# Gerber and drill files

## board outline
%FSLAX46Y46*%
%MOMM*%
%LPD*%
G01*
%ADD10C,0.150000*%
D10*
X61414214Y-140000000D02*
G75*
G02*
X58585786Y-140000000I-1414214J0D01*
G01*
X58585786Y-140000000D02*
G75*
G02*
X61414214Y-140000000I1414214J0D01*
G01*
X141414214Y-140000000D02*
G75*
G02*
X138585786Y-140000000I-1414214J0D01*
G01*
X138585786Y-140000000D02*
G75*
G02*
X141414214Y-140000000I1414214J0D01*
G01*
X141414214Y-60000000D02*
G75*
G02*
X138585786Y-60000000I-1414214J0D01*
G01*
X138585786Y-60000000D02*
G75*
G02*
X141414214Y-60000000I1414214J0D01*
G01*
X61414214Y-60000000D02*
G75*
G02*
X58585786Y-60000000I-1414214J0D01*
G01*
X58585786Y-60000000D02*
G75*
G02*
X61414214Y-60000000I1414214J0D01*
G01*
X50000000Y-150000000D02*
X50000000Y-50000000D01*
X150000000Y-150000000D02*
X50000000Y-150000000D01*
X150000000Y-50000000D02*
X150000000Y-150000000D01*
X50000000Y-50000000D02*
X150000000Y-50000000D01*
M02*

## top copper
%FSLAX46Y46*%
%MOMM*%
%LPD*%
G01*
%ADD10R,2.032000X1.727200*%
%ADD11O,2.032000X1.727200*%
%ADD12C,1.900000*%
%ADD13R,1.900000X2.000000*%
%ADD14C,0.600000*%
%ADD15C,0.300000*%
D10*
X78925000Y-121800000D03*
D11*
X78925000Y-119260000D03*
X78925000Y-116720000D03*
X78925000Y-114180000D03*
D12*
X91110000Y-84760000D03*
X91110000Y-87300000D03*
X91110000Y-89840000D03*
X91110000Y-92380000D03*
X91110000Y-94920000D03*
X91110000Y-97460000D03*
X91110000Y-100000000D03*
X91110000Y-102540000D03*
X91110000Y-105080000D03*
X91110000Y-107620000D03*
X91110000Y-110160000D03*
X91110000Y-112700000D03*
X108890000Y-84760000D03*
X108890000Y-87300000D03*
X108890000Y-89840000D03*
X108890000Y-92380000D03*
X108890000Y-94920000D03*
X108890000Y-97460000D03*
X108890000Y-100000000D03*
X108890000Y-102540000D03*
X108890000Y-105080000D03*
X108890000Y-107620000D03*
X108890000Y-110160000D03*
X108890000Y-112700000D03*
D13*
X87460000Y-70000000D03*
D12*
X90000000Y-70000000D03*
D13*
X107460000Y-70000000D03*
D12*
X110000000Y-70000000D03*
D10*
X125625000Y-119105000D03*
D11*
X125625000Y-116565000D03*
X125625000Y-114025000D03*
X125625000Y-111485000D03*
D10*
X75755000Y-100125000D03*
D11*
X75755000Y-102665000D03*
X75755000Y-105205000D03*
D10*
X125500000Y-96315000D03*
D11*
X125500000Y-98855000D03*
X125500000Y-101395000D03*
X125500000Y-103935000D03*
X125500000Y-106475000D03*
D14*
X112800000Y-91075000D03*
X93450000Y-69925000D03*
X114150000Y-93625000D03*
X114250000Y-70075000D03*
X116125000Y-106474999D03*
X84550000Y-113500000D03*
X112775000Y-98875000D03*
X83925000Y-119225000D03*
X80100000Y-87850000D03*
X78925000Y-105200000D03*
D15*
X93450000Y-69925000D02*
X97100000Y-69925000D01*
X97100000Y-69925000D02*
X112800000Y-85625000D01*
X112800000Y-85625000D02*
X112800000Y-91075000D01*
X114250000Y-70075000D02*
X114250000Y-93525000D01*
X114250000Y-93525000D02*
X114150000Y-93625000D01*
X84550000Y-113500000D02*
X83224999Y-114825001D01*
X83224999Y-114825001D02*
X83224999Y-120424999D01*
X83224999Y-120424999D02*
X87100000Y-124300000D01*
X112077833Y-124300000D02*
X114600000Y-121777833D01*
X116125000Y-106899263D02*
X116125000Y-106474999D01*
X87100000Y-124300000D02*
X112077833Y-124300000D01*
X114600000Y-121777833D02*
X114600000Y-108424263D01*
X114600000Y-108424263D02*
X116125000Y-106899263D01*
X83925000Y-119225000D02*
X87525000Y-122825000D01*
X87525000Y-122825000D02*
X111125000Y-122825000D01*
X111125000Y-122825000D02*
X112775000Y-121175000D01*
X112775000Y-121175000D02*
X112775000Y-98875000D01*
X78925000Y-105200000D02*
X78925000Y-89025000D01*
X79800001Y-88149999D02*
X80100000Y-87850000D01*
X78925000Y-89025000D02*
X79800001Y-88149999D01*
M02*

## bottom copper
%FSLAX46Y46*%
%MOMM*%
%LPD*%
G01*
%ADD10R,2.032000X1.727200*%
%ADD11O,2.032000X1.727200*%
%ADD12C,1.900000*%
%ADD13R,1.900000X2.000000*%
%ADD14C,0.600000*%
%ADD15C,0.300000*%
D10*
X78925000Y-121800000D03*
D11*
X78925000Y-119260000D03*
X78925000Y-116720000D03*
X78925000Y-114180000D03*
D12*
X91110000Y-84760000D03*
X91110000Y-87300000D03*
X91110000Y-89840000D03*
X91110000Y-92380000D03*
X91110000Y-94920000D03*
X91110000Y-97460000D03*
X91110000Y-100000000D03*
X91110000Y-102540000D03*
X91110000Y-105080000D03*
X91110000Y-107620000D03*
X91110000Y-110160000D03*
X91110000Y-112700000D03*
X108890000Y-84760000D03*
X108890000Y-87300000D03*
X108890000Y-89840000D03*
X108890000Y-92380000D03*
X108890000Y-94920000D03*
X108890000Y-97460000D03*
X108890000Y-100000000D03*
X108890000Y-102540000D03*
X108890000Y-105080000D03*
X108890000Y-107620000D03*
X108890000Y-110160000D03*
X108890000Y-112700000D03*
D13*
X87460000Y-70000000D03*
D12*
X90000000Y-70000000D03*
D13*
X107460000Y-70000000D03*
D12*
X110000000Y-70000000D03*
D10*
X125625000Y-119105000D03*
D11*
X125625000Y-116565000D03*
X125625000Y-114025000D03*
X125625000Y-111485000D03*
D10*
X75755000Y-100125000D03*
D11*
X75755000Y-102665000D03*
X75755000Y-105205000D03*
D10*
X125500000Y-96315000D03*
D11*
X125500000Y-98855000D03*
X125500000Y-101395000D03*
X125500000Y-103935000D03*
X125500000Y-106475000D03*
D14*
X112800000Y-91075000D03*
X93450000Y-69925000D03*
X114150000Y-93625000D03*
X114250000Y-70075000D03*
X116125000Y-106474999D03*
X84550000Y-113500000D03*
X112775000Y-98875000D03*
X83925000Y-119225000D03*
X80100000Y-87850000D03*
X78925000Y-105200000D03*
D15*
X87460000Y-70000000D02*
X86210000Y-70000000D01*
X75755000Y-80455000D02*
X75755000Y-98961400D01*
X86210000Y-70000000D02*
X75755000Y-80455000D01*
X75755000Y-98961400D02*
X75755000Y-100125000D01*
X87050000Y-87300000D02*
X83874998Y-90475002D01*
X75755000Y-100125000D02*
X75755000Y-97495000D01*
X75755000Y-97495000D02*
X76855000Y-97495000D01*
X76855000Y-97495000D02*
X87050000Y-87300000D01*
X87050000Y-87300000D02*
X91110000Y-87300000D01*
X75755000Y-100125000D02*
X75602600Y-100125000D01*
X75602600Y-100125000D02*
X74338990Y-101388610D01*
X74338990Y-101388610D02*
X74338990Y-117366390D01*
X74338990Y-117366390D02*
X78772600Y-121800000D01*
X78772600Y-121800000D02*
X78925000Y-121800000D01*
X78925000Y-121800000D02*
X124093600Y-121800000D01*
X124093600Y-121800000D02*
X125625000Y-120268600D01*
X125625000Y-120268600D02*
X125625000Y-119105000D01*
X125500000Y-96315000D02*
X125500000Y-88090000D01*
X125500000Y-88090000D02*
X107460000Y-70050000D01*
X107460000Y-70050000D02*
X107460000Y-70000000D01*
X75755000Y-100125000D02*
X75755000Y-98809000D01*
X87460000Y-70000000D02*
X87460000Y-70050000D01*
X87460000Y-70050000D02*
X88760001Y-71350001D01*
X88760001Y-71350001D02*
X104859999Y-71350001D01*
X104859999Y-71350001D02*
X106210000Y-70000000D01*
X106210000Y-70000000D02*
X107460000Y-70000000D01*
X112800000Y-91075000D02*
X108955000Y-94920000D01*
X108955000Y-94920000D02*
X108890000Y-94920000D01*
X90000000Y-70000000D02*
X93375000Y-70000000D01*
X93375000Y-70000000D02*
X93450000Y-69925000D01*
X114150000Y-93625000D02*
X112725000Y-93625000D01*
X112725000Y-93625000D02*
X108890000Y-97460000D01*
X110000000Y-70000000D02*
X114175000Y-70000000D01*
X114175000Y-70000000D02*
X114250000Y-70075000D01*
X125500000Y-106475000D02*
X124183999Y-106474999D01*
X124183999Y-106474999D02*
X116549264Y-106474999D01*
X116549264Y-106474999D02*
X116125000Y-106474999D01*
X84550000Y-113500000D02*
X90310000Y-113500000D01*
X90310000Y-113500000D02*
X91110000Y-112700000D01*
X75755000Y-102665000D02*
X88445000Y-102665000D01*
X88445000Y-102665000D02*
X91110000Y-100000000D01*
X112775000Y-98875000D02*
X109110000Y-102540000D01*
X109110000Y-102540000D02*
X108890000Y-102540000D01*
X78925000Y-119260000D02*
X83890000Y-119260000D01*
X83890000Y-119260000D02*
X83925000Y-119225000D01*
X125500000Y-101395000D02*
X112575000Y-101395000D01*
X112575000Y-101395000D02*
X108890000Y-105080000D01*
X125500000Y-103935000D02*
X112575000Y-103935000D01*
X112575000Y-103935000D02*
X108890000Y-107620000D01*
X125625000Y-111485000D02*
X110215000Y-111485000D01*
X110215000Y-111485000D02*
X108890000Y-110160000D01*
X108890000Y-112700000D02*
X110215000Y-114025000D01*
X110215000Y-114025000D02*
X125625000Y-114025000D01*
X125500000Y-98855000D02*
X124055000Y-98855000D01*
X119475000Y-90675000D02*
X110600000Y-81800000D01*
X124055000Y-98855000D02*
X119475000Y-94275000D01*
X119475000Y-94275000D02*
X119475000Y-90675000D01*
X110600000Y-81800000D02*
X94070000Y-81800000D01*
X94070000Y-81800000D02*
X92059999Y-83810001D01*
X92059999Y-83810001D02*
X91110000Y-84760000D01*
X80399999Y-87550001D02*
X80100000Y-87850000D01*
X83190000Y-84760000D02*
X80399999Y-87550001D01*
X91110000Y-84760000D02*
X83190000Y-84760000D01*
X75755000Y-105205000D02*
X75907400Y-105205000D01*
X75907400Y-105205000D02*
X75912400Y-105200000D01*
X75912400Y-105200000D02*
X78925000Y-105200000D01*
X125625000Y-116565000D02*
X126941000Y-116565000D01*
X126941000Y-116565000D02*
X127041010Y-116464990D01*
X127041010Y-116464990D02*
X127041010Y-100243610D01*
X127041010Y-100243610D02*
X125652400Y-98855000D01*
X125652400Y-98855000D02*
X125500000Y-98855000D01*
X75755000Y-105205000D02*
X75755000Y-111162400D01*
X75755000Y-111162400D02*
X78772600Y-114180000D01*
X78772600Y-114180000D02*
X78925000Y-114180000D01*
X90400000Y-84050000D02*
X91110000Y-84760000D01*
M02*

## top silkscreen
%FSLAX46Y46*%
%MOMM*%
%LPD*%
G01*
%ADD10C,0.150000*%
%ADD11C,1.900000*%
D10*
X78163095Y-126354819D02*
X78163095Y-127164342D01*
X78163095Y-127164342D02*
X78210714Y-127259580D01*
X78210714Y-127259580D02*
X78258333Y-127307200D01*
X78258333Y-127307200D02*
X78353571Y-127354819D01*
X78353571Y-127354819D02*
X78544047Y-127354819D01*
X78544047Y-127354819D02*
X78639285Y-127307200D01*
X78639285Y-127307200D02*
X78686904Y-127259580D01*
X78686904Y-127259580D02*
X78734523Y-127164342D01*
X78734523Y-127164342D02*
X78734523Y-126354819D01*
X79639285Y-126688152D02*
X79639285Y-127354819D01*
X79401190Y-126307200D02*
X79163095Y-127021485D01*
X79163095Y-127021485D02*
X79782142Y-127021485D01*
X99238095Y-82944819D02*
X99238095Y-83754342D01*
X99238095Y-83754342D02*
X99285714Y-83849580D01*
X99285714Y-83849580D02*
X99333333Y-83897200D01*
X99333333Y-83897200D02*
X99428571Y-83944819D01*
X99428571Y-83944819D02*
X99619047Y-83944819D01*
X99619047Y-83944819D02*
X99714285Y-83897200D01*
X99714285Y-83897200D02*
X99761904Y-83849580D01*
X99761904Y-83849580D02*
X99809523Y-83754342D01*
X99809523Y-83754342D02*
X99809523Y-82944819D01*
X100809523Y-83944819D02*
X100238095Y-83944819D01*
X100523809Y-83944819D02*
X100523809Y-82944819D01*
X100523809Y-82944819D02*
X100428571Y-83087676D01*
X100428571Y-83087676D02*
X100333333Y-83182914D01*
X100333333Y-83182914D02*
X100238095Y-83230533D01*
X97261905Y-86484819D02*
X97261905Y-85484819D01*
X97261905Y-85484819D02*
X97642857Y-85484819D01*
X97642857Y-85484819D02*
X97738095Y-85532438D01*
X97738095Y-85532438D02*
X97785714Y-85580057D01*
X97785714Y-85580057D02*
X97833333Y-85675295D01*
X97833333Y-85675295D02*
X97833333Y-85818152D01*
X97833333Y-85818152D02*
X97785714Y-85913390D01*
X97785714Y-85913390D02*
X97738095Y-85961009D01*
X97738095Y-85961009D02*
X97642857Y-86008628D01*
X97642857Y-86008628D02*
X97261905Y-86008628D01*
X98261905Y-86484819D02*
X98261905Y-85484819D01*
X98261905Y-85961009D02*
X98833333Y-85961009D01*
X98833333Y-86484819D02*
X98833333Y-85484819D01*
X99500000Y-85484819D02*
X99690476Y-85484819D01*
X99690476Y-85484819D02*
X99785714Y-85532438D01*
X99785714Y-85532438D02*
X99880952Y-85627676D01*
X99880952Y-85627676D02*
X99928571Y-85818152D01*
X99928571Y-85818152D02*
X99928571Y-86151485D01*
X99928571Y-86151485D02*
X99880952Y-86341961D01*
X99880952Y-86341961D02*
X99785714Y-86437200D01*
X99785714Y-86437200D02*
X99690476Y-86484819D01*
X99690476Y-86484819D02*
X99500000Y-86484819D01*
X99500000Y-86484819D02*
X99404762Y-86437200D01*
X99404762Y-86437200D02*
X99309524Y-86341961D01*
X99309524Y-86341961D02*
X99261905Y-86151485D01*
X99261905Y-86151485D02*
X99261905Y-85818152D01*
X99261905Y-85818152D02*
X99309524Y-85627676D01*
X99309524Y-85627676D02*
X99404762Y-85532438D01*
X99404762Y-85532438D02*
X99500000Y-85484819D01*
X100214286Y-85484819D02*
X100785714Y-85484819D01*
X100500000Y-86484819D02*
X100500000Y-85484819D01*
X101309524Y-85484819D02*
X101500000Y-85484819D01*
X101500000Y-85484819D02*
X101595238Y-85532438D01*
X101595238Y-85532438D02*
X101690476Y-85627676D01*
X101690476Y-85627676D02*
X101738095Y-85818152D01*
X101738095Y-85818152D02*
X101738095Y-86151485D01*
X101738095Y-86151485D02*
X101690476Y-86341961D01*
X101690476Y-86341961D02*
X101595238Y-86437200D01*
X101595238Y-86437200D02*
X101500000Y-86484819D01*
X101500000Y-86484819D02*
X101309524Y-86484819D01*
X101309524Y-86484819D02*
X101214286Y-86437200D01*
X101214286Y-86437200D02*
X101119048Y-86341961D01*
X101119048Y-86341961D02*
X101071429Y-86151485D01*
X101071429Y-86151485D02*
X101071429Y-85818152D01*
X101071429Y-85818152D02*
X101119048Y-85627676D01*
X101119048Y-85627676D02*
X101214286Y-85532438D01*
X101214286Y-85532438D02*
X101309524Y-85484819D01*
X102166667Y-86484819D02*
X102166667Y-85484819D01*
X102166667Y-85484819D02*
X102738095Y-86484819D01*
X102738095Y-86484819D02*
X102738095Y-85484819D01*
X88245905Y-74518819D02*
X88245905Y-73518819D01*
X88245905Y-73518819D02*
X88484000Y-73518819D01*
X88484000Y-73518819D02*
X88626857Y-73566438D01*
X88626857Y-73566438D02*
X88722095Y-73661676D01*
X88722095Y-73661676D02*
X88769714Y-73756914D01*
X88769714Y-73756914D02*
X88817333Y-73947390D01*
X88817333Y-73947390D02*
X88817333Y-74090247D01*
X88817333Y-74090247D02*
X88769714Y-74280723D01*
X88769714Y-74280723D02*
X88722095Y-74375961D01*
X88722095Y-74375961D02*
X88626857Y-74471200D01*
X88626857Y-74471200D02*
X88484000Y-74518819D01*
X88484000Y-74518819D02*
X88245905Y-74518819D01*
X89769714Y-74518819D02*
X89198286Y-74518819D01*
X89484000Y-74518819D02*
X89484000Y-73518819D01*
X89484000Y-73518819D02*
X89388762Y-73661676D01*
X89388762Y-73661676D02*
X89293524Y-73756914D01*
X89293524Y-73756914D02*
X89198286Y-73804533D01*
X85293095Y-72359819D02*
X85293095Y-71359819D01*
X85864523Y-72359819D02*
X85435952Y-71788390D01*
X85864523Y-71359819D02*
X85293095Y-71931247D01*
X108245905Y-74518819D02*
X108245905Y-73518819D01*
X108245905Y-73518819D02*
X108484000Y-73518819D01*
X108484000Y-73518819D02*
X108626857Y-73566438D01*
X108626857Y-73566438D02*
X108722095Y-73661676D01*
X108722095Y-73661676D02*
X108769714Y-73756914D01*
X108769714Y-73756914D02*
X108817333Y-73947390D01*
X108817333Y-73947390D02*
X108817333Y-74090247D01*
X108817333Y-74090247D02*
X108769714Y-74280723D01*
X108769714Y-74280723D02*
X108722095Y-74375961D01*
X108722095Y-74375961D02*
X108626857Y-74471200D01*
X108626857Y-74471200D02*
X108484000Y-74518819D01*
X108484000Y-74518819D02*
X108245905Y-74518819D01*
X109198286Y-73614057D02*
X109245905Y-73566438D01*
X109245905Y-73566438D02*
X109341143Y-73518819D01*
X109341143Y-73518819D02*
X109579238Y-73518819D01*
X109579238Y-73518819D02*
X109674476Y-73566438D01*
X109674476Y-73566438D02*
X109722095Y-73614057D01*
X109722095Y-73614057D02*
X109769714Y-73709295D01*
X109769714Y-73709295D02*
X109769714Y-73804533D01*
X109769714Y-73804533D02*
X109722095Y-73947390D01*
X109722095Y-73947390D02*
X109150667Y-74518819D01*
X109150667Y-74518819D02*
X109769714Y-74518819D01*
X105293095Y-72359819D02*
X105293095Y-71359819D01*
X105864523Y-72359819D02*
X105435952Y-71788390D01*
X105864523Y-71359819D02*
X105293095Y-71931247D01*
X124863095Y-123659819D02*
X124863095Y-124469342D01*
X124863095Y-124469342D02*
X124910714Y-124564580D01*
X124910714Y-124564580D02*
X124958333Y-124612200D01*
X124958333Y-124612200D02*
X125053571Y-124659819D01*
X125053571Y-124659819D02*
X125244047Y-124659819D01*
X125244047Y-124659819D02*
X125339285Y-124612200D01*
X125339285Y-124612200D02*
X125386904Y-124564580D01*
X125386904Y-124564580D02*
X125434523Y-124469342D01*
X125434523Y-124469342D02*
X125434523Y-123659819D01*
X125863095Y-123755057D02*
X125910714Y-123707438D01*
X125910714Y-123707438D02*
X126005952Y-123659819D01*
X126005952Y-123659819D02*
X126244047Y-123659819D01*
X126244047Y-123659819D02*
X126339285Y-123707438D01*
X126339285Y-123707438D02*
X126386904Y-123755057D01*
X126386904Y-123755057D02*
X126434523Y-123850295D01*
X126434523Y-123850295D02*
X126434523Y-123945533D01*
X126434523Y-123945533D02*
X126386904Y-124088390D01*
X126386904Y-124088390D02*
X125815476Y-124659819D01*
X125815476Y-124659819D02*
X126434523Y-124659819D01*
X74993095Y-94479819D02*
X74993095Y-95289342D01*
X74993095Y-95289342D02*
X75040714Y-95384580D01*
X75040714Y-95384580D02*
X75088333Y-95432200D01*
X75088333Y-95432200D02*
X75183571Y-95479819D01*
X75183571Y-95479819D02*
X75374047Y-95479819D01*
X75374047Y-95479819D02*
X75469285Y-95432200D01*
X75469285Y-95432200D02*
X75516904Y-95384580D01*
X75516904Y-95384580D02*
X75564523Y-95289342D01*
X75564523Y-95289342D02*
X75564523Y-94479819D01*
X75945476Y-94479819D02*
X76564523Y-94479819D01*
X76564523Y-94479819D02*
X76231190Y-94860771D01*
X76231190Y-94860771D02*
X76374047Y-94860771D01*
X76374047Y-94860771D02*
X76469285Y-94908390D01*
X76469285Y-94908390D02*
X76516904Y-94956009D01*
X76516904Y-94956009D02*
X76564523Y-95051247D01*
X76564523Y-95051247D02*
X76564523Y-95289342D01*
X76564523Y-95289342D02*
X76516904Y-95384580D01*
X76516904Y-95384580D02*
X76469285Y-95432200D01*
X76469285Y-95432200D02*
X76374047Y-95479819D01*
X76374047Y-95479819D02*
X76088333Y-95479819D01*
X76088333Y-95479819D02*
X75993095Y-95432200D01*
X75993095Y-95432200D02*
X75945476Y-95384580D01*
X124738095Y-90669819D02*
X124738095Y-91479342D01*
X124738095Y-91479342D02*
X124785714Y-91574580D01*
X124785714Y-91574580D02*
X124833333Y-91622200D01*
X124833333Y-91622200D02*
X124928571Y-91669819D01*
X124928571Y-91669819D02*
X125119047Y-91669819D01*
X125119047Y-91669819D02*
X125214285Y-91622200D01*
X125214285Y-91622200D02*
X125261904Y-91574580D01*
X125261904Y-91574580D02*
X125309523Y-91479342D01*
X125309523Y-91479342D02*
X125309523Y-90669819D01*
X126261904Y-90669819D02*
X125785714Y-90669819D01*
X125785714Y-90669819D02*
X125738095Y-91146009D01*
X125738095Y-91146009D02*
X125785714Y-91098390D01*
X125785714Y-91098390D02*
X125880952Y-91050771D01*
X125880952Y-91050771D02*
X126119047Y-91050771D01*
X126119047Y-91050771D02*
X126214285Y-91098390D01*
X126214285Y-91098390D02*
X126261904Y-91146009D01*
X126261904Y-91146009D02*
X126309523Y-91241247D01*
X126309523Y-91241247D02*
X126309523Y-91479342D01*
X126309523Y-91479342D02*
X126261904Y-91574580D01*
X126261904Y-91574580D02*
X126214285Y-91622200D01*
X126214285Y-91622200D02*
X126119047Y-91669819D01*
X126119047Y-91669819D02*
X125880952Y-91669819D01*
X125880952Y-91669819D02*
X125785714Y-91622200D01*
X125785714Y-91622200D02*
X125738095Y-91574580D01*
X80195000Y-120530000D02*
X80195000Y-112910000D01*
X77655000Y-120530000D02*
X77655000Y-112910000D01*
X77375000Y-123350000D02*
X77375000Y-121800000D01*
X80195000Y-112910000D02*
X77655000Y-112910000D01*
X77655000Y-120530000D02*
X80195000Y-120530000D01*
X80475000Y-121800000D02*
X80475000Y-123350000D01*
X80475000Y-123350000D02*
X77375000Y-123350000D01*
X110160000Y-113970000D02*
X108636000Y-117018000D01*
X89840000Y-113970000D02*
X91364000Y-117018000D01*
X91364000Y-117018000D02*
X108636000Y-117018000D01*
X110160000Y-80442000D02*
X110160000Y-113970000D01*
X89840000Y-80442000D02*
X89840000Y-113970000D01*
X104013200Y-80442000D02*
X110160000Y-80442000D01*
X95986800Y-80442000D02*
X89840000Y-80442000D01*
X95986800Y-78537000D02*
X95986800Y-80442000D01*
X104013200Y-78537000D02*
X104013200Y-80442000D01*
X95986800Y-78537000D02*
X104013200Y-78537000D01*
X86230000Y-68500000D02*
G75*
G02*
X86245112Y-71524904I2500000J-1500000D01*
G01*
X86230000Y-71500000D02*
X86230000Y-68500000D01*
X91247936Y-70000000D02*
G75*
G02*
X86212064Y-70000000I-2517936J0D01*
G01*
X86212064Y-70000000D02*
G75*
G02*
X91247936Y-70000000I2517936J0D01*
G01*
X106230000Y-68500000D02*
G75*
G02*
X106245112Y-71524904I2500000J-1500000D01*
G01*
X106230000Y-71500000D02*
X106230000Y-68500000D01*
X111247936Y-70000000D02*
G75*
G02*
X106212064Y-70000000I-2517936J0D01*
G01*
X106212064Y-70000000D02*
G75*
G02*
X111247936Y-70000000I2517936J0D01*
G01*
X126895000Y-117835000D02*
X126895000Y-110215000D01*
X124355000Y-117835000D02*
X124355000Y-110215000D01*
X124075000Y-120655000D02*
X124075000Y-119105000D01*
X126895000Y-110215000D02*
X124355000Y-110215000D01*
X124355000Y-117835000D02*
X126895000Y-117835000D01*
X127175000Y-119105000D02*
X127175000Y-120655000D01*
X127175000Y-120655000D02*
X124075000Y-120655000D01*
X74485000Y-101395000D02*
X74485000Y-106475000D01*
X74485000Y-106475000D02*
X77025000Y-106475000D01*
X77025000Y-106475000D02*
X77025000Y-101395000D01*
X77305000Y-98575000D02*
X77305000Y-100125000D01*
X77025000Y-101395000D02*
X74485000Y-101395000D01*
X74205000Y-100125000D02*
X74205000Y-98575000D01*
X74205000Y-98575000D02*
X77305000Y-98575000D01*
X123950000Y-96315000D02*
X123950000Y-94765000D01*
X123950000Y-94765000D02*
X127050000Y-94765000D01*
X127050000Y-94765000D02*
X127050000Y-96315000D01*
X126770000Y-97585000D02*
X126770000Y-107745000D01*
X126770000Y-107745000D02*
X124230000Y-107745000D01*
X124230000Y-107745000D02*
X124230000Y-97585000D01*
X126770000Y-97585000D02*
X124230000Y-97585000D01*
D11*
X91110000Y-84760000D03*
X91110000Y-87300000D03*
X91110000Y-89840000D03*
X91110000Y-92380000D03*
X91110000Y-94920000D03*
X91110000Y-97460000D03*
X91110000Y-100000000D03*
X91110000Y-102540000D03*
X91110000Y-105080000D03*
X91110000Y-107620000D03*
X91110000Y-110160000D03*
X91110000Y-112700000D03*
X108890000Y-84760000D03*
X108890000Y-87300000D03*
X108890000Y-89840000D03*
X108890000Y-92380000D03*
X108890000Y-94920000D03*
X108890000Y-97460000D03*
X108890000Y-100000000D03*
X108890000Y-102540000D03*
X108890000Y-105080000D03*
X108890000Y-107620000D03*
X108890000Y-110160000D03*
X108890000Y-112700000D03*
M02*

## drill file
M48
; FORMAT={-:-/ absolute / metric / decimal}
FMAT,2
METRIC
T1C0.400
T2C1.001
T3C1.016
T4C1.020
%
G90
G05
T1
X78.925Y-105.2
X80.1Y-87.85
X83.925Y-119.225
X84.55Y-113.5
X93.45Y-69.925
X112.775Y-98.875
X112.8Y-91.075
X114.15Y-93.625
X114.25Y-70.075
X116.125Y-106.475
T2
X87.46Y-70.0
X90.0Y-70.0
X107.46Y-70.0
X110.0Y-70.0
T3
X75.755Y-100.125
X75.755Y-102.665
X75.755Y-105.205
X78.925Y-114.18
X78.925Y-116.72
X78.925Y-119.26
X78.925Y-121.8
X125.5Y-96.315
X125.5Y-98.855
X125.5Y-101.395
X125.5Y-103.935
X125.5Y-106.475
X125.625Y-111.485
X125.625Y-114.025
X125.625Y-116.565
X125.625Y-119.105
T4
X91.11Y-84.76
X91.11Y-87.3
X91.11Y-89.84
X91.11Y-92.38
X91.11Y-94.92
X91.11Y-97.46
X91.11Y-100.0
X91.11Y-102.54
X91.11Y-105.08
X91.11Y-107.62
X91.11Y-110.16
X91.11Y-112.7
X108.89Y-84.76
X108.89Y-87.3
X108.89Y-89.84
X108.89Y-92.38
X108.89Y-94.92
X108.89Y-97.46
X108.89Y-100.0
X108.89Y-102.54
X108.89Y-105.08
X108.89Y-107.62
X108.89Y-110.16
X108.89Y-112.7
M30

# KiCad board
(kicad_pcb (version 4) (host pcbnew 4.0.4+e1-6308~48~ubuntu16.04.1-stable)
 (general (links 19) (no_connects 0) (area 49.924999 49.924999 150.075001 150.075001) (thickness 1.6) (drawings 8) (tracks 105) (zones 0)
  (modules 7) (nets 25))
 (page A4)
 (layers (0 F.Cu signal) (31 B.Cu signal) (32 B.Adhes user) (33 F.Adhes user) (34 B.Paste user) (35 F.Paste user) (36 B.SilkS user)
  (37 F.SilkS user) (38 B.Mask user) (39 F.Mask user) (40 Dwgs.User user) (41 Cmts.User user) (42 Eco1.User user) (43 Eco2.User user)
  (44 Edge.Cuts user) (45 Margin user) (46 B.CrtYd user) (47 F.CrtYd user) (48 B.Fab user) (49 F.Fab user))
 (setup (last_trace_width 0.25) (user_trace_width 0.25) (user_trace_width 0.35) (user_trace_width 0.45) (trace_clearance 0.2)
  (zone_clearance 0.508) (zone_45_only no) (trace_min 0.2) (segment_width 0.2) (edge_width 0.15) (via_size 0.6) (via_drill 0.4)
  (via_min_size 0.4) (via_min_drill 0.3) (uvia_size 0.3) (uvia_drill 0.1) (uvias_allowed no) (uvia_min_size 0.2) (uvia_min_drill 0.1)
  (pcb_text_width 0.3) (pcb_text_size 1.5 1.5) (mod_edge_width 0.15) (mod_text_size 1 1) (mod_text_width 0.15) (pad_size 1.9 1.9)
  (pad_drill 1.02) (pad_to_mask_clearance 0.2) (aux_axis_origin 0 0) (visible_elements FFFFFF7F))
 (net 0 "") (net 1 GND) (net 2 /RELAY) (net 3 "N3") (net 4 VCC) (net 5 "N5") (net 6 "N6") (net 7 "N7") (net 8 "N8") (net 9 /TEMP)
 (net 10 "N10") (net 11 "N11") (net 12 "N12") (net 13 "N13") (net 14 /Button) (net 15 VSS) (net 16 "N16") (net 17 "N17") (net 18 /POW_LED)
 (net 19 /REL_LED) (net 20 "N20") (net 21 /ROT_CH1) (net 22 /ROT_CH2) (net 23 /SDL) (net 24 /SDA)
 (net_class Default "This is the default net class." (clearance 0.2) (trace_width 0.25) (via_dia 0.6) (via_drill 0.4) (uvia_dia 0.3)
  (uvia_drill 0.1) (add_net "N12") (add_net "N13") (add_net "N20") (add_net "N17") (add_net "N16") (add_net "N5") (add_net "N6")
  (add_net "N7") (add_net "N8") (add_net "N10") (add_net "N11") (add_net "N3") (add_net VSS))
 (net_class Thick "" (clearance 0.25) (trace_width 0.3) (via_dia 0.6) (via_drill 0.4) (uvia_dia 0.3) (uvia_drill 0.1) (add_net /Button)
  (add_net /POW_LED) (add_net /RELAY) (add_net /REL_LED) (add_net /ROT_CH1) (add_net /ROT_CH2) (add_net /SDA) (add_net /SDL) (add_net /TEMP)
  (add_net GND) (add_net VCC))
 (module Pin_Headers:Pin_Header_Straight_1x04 (layer F.Cu) (at 78.925 121.8 180)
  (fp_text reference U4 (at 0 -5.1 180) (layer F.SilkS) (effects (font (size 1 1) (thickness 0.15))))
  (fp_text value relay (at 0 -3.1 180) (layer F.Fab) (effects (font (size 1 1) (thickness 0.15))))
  (fp_line (start -1.27 1.27) (end -1.27 8.89) (layer F.SilkS) (width 0.15))
  (fp_line (start 1.27 1.27) (end 1.27 8.89) (layer F.SilkS) (width 0.15))
  (fp_line (start 1.55 -1.55) (end 1.55 0) (layer F.SilkS) (width 0.15))
  (fp_line (start -1.27 8.89) (end 1.27 8.89) (layer F.SilkS) (width 0.15))
  (fp_line (start 1.27 1.27) (end -1.27 1.27) (layer F.SilkS) (width 0.15))
  (fp_line (start -1.55 0) (end -1.55 -1.55) (layer F.SilkS) (width 0.15))
  (fp_line (start -1.55 -1.55) (end 1.55 -1.55) (layer F.SilkS) (width 0.15))
  (pad 1 thru_hole rect (at 0 0 180) (size 2.032 1.7272) (drill 1.016) (layers *.Cu *.Mask) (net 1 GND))
  (pad 2 thru_hole oval (at 0 2.54 180) (size 2.032 1.7272) (drill 1.016) (layers *.Cu *.Mask) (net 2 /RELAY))
  (pad 3 thru_hole oval (at 0 5.08 180) (size 2.032 1.7272) (drill 1.016) (layers *.Cu *.Mask) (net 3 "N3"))
  (pad 4 thru_hole oval (at 0 7.62 180) (size 2.032 1.7272) (drill 1.016) (layers *.Cu *.Mask) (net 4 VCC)))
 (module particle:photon (layer F.Cu) (at 100 100)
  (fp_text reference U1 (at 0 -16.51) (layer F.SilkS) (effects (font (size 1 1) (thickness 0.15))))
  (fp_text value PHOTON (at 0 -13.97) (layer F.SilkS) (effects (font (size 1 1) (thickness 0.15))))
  (fp_line (start 10.16 13.97) (end 8.636 17.018) (layer F.SilkS) (width 0.15))
  (fp_line (start -10.16 13.97) (end -8.636 17.018) (layer F.SilkS) (width 0.15))
  (fp_line (start -8.636 17.018) (end 8.636 17.018) (layer F.SilkS) (width 0.15))
  (fp_line (start 10.16 -19.558) (end 10.16 13.97) (layer F.SilkS) (width 0.15))
  (fp_line (start -10.16 -19.558) (end -10.16 13.97) (layer F.SilkS) (width 0.15))
  (fp_line (start 4.0132 -19.558) (end 10.16 -19.558) (layer F.SilkS) (width 0.15))
  (fp_line (start -4.0132 -19.558) (end -10.16 -19.558) (layer F.SilkS) (width 0.15))
  (fp_line (start -4.0132 -21.463) (end -4.0132 -19.558) (layer F.SilkS) (width 0.15))
  (fp_line (start 4.0132 -21.463) (end 4.0132 -19.558) (layer F.SilkS) (width 0.15))
  (fp_line (start -4.0132 -21.463) (end 4.0132 -21.463) (layer F.SilkS) (width 0.15))
  (pad 1 thru_hole circle (at -8.89 -15.24) (size 1.9 1.9) (drill 1.02) (layers *.Cu *.Mask F.SilkS) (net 4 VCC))
  (pad 2 thru_hole circle (at -8.89 -12.7) (size 1.9 1.9) (drill 1.02) (layers *.Cu *.Mask F.SilkS) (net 1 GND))
  (pad 3 thru_hole circle (at -8.89 -10.16) (size 1.9 1.9) (drill 1.02) (layers *.Cu *.Mask F.SilkS) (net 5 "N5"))
  (pad 4 thru_hole circle (at -8.89 -7.62) (size 1.9 1.9) (drill 1.02) (layers *.Cu *.Mask F.SilkS) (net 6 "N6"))
  (pad 5 thru_hole circle (at -8.89 -5.08) (size 1.9 1.9) (drill 1.02) (layers *.Cu *.Mask F.SilkS) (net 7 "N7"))
  (pad 6 thru_hole circle (at -8.89 -2.54) (size 1.9 1.9) (drill 1.02) (layers *.Cu *.Mask F.SilkS) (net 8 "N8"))
  (pad 7 thru_hole circle (at -8.89 0) (size 1.9 1.9) (drill 1.02) (layers *.Cu *.Mask F.SilkS) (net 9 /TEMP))
  (pad 8 thru_hole circle (at -8.89 2.54) (size 1.9 1.9) (drill 1.02) (layers *.Cu *.Mask F.SilkS) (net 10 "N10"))
  (pad 9 thru_hole circle (at -8.89 5.08) (size 1.9 1.9) (drill 1.02) (layers *.Cu *.Mask F.SilkS) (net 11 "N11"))
  (pad 10 thru_hole circle (at -8.89 7.62) (size 1.9 1.9) (drill 1.02) (layers *.Cu *.Mask F.SilkS) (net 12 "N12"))
  (pad 11 thru_hole circle (at -8.89 10.16) (size 1.9 1.9) (drill 1.02) (layers *.Cu *.Mask F.SilkS) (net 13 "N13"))
  (pad 12 thru_hole circle (at -8.89 12.7) (size 1.9 1.9) (drill 1.02) (layers *.Cu *.Mask F.SilkS) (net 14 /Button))
  (pad 24 thru_hole circle (at 8.89 -15.24) (size 1.9 1.9) (drill 1.02) (layers *.Cu *.Mask F.SilkS) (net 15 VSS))
  (pad 23 thru_hole circle (at 8.89 -12.7) (size 1.9 1.9) (drill 1.02) (layers *.Cu *.Mask F.SilkS) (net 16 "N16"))
  (pad 22 thru_hole circle (at 8.89 -10.16) (size 1.9 1.9) (drill 1.02) (layers *.Cu *.Mask F.SilkS) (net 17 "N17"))
  (pad 21 thru_hole circle (at 8.89 -7.62) (size 1.9 1.9) (drill 1.02) (layers *.Cu *.Mask F.SilkS))
  (pad 20 thru_hole circle (at 8.89 -5.08) (size 1.9 1.9) (drill 1.02) (layers *.Cu *.Mask F.SilkS) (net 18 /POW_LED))
  (pad 19 thru_hole circle (at 8.89 -2.54) (size 1.9 1.9) (drill 1.02) (layers *.Cu *.Mask F.SilkS) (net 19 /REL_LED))
  (pad 18 thru_hole circle (at 8.89 0) (size 1.9 1.9) (drill 1.02) (layers *.Cu *.Mask F.SilkS) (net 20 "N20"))
  (pad 17 thru_hole circle (at 8.89 2.54) (size 1.9 1.9) (drill 1.02) (layers *.Cu *.Mask F.SilkS) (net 2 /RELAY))
  (pad 16 thru_hole circle (at 8.89 5.08) (size 1.9 1.9) (drill 1.02) (layers *.Cu *.Mask F.SilkS) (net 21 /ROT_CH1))
  (pad 15 thru_hole circle (at 8.89 7.62) (size 1.9 1.9) (drill 1.02) (layers *.Cu *.Mask F.SilkS) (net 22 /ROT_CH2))
  (pad 14 thru_hole circle (at 8.89 10.16) (size 1.9 1.9) (drill 1.02) (layers *.Cu *.Mask F.SilkS) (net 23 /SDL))
  (pad 13 thru_hole circle (at 8.89 12.7) (size 1.9 1.9) (drill 1.02) (layers *.Cu *.Mask F.SilkS) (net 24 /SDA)))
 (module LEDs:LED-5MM (layer F.Cu) (at 87.46 70)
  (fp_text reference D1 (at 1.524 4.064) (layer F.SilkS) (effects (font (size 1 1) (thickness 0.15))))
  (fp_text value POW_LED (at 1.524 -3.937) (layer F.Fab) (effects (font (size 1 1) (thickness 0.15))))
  (fp_arc (start 1.27 0) (end -1.23 -1.5) (angle 297.5) (layer F.SilkS) (width 0.15))
  (fp_line (start -1.23 1.5) (end -1.23 -1.5) (layer F.SilkS) (width 0.15))
  (fp_circle (center 1.27 0) (end 0.97 -2.5) (layer F.SilkS) (width 0.15))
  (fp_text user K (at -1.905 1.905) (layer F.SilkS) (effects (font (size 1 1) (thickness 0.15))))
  (pad 1 thru_hole rect (at 0 0 90) (size 2 1.9) (drill 1.00076) (layers *.Cu *.Mask) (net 1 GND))
  (pad 2 thru_hole circle (at 2.54 0) (size 1.9 1.9) (drill 1.00076) (layers *.Cu *.Mask) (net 18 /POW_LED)))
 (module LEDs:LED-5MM (layer F.Cu) (at 107.46 70)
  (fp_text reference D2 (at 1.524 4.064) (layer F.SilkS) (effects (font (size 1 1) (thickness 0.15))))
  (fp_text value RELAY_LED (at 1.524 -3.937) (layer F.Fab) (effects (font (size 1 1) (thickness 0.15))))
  (fp_arc (start 1.27 0) (end -1.23 -1.5) (angle 297.5) (layer F.SilkS) (width 0.15))
  (fp_line (start -1.23 1.5) (end -1.23 -1.5) (layer F.SilkS) (width 0.15))
  (fp_circle (center 1.27 0) (end 0.97 -2.5) (layer F.SilkS) (width 0.15))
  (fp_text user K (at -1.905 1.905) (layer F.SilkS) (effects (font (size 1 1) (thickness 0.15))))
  (pad 1 thru_hole rect (at 0 0 90) (size 2 1.9) (drill 1.00076) (layers *.Cu *.Mask) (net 1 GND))
  (pad 2 thru_hole circle (at 2.54 0) (size 1.9 1.9) (drill 1.00076) (layers *.Cu *.Mask) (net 19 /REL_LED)))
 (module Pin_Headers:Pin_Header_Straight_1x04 (layer F.Cu) (at 125.625 119.105 180)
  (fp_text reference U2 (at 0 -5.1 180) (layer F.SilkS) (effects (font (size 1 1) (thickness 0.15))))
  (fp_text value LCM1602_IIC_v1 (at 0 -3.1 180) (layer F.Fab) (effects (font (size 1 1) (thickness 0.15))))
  (fp_line (start -1.27 1.27) (end -1.27 8.89) (layer F.SilkS) (width 0.15))
  (fp_line (start 1.27 1.27) (end 1.27 8.89) (layer F.SilkS) (width 0.15))
  (fp_line (start 1.55 -1.55) (end 1.55 0) (layer F.SilkS) (width 0.15))
  (fp_line (start -1.27 8.89) (end 1.27 8.89) (layer F.SilkS) (width 0.15))
  (fp_line (start 1.27 1.27) (end -1.27 1.27) (layer F.SilkS) (width 0.15))
  (fp_line (start -1.55 0) (end -1.55 -1.55) (layer F.SilkS) (width 0.15))
  (fp_line (start -1.55 -1.55) (end 1.55 -1.55) (layer F.SilkS) (width 0.15))
  (pad 1 thru_hole rect (at 0 0 180) (size 2.032 1.7272) (drill 1.016) (layers *.Cu *.Mask) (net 1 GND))
  (pad 2 thru_hole oval (at 0 2.54 180) (size 2.032 1.7272) (drill 1.016) (layers *.Cu *.Mask) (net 4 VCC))
  (pad 3 thru_hole oval (at 0 5.08 180) (size 2.032 1.7272) (drill 1.016) (layers *.Cu *.Mask) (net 24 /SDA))
  (pad 4 thru_hole oval (at 0 7.62 180) (size 2.032 1.7272) (drill 1.016) (layers *.Cu *.Mask) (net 23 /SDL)))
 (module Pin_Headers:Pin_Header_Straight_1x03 (layer F.Cu) (at 75.755 100.125)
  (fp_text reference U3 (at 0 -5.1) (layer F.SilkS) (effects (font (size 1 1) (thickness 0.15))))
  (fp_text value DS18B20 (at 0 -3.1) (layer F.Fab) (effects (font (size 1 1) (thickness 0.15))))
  (fp_line (start -1.27 1.27) (end -1.27 6.35) (layer F.SilkS) (width 0.15))
  (fp_line (start -1.27 6.35) (end 1.27 6.35) (layer F.SilkS) (width 0.15))
  (fp_line (start 1.27 6.35) (end 1.27 1.27) (layer F.SilkS) (width 0.15))
  (fp_line (start 1.55 -1.55) (end 1.55 0) (layer F.SilkS) (width 0.15))
  (fp_line (start 1.27 1.27) (end -1.27 1.27) (layer F.SilkS) (width 0.15))
  (fp_line (start -1.55 0) (end -1.55 -1.55) (layer F.SilkS) (width 0.15))
  (fp_line (start -1.55 -1.55) (end 1.55 -1.55) (layer F.SilkS) (width 0.15))
  (pad 1 thru_hole rect (at 0 0) (size 2.032 1.7272) (drill 1.016) (layers *.Cu *.Mask) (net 1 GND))
  (pad 2 thru_hole oval (at 0 2.54) (size 2.032 1.7272) (drill 1.016) (layers *.Cu *.Mask) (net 9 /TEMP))
  (pad 3 thru_hole oval (at 0 5.08) (size 2.032 1.7272) (drill 1.016) (layers *.Cu *.Mask) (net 4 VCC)))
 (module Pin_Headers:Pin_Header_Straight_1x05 (layer F.Cu) (at 125.5 96.315)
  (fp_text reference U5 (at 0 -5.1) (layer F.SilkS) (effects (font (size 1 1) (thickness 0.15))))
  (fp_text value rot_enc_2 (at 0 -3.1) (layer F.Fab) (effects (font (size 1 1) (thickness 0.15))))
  (fp_line (start -1.55 0) (end -1.55 -1.55) (layer F.SilkS) (width 0.15))
  (fp_line (start -1.55 -1.55) (end 1.55 -1.55) (layer F.SilkS) (width 0.15))
  (fp_line (start 1.55 -1.55) (end 1.55 0) (layer F.SilkS) (width 0.15))
  (fp_line (start 1.27 1.27) (end 1.27 11.43) (layer F.SilkS) (width 0.15))
  (fp_line (start 1.27 11.43) (end -1.27 11.43) (layer F.SilkS) (width 0.15))
  (fp_line (start -1.27 11.43) (end -1.27 1.27) (layer F.SilkS) (width 0.15))
  (fp_line (start 1.27 1.27) (end -1.27 1.27) (layer F.SilkS) (width 0.15))
  (pad 1 thru_hole rect (at 0 0) (size 2.032 1.7272) (drill 1.016) (layers *.Cu *.Mask) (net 1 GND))
  (pad 2 thru_hole oval (at 0 2.54) (size 2.032 1.7272) (drill 1.016) (layers *.Cu *.Mask) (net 4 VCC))
  (pad 3 thru_hole oval (at 0 5.08) (size 2.032 1.7272) (drill 1.016) (layers *.Cu *.Mask) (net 21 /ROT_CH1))
  (pad 4 thru_hole oval (at 0 7.62) (size 2.032 1.7272) (drill 1.016) (layers *.Cu *.Mask) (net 22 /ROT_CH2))
  (pad 5 thru_hole oval (at 0 10.16) (size 2.032 1.7272) (drill 1.016) (layers *.Cu *.Mask) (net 14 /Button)))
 (gr_circle (center 60 140) (end 61 141) (layer Edge.Cuts) (width 0.15))
 (gr_circle (center 140 140) (end 141 141) (layer Edge.Cuts) (width 0.15))
 (gr_circle (center 140 60) (end 141 61) (layer Edge.Cuts) (width 0.15))
 (gr_circle (center 60 60) (end 61 61) (layer Edge.Cuts) (width 0.15))
 (gr_line (start 50 150) (end 50 50) (angle 90) (layer Edge.Cuts) (width 0.15))
 (gr_line (start 150 150) (end 50 150) (angle 90) (layer Edge.Cuts) (width 0.15))
 (gr_line (start 150 50) (end 150 150) (angle 90) (layer Edge.Cuts) (width 0.15))
 (gr_line (start 50 50) (end 150 50) (angle 90) (layer Edge.Cuts) (width 0.15))
 (segment (start 87.46 70) (end 86.21 70) (width 0.3) (layer B.Cu) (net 1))
 (segment (start 75.755 80.455) (end 75.755 98.9614) (width 0.3) (layer B.Cu) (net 1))
 (segment (start 86.21 70) (end 75.755 80.455) (width 0.3) (layer B.Cu) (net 1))
 (segment (start 75.755 98.9614) (end 75.755 100.125) (width 0.3) (layer B.Cu) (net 1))
 (segment (start 87.05 87.3) (end 83.874998 90.475002) (width 0.3) (layer B.Cu) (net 1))
 (segment (start 75.755 100.125) (end 75.755 97.495) (width 0.3) (layer B.Cu) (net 1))
 (segment (start 75.755 97.495) (end 76.855 97.495) (width 0.3) (layer B.Cu) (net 1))
 (segment (start 76.855 97.495) (end 87.05 87.3) (width 0.3) (layer B.Cu) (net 1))
 (segment (start 87.05 87.3) (end 91.11 87.3) (width 0.3) (layer B.Cu) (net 1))
 (segment (start 75.755 100.125) (end 75.6026 100.125) (width 0.3) (layer B.Cu) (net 1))
 (segment (start 75.6026 100.125) (end 74.33899 101.38861) (width 0.3) (layer B.Cu) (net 1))
 (segment (start 74.33899 101.38861) (end 74.33899 117.36639) (width 0.3) (layer B.Cu) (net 1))
 (segment (start 74.33899 117.36639) (end 78.7726 121.8) (width 0.3) (layer B.Cu) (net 1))
 (segment (start 78.7726 121.8) (end 78.925 121.8) (width 0.3) (layer B.Cu) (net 1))
 (segment (start 78.925 121.8) (end 124.0936 121.8) (width 0.3) (layer B.Cu) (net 1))
 (segment (start 124.0936 121.8) (end 125.625 120.2686) (width 0.3) (layer B.Cu) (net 1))
 (segment (start 125.625 120.2686) (end 125.625 119.105) (width 0.3) (layer B.Cu) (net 1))
 (segment (start 125.5 96.315) (end 125.5 88.09) (width 0.3) (layer B.Cu) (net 1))
 (segment (start 125.5 88.09) (end 107.46 70.05) (width 0.3) (layer B.Cu) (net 1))
 (segment (start 107.46 70.05) (end 107.46 70) (width 0.3) (layer B.Cu) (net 1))
 (segment (start 75.755 100.125) (end 75.755 98.809) (width 0.3) (layer B.Cu) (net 1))
 (segment (start 87.46 70) (end 87.46 70.05) (width 0.3) (layer B.Cu) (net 1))
 (segment (start 87.46 70.05) (end 88.760001 71.350001) (width 0.3) (layer B.Cu) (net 1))
 (segment (start 88.760001 71.350001) (end 104.859999 71.350001) (width 0.3) (layer B.Cu) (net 1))
 (segment (start 104.859999 71.350001) (end 106.21 70) (width 0.3) (layer B.Cu) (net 1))
 (segment (start 106.21 70) (end 107.46 70) (width 0.3) (layer B.Cu) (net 1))
 (segment (start 93.45 69.925) (end 97.1 69.925) (width 0.3) (layer F.Cu) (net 18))
 (segment (start 97.1 69.925) (end 112.8 85.625) (width 0.3) (layer F.Cu) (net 18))
 (segment (start 112.8 85.625) (end 112.8 91.075) (width 0.3) (layer F.Cu) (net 18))
 (segment (start 112.8 91.075) (end 108.955 94.92) (width 0.3) (layer B.Cu) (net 18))
 (segment (start 108.955 94.92) (end 108.89 94.92) (width 0.3) (layer B.Cu) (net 18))
 (via (at 112.8 91.075) (size 0.6) (drill 0.4) (layers F.Cu B.Cu) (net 18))
 (segment (start 90 70) (end 93.375 70) (width 0.3) (layer B.Cu) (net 18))
 (segment (start 93.375 70) (end 93.45 69.925) (width 0.3) (layer B.Cu) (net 18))
 (via (at 93.45 69.925) (size 0.6) (drill 0.4) (layers F.Cu B.Cu) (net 18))
 (segment (start 114.15 93.625) (end 112.725 93.625) (width 0.3) (layer B.Cu) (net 19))
 (segment (start 112.725 93.625) (end 108.89 97.46) (width 0.3) (layer B.Cu) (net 19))
 (segment (start 114.25 70.075) (end 114.25 93.525) (width 0.3) (layer F.Cu) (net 19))
 (segment (start 114.25 93.525) (end 114.15 93.625) (width 0.3) (layer F.Cu) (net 19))
 (via (at 114.15 93.625) (size 0.6) (drill 0.4) (layers F.Cu B.Cu) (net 19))
 (segment (start 110 70) (end 114.175 70) (width 0.3) (layer B.Cu) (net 19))
 (segment (start 114.175 70) (end 114.25 70.075) (width 0.3) (layer B.Cu) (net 19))
 (via (at 114.25 70.075) (size 0.6) (drill 0.4) (layers F.Cu B.Cu) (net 19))
 (segment (start 84.55 113.5) (end 83.224999 114.825001) (width 0.3) (layer F.Cu) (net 14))
 (segment (start 83.224999 114.825001) (end 83.224999 120.424999) (width 0.3) (layer F.Cu) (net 14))
 (segment (start 83.224999 120.424999) (end 87.1 124.3) (width 0.3) (layer F.Cu) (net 14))
 (segment (start 112.077833 124.3) (end 114.6 121.777833) (width 0.3) (layer F.Cu) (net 14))
 (segment (start 116.125 106.899263) (end 116.125 106.474999) (width 0.3) (layer F.Cu) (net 14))
 (segment (start 87.1 124.3) (end 112.077833 124.3) (width 0.3) (layer F.Cu) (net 14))
 (segment (start 114.6 121.777833) (end 114.6 108.424263) (width 0.3) (layer F.Cu) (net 14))
 (segment (start 114.6 108.424263) (end 116.125 106.899263) (width 0.3) (layer F.Cu) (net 14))
 (segment (start 125.5 106.475) (end 124.183999 106.474999) (width 0.3) (layer B.Cu) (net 14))
 (segment (start 124.183999 106.474999) (end 116.549264 106.474999) (width 0.3) (layer B.Cu) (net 14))
 (segment (start 116.549264 106.474999) (end 116.125 106.474999) (width 0.3) (layer B.Cu) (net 14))
 (via (at 116.125 106.474999) (size 0.6) (drill 0.4) (layers F.Cu B.Cu) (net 14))
 (segment (start 84.55 113.5) (end 90.31 113.5) (width 0.3) (layer B.Cu) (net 14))
 (segment (start 90.31 113.5) (end 91.11 112.7) (width 0.3) (layer B.Cu) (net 14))
 (via (at 84.55 113.5) (size 0.6) (drill 0.4) (layers F.Cu B.Cu) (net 14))
 (segment (start 75.755 102.665) (end 88.445 102.665) (width 0.3) (layer B.Cu) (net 9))
 (segment (start 88.445 102.665) (end 91.11 100) (width 0.3) (layer B.Cu) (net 9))
 (segment (start 83.925 119.225) (end 87.525 122.825) (width 0.3) (layer F.Cu) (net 2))
 (segment (start 87.525 122.825) (end 111.125 122.825) (width 0.3) (layer F.Cu) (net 2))
 (segment (start 111.125 122.825) (end 112.775 121.175) (width 0.3) (layer F.Cu) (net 2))
 (segment (start 112.775 121.175) (end 112.775 98.875) (width 0.3) (layer F.Cu) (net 2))
 (segment (start 112.775 98.875) (end 109.11 102.54) (width 0.3) (layer B.Cu) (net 2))
 (segment (start 109.11 102.54) (end 108.89 102.54) (width 0.3) (layer B.Cu) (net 2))
 (via (at 112.775 98.875) (size 0.6) (drill 0.4) (layers F.Cu B.Cu) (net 2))
 (segment (start 78.925 119.26) (end 83.89 119.26) (width 0.3) (layer B.Cu) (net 2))
 (segment (start 83.89 119.26) (end 83.925 119.225) (width 0.3) (layer B.Cu) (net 2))
 (via (at 83.925 119.225) (size 0.6) (drill 0.4) (layers F.Cu B.Cu) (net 2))
 (segment (start 125.5 101.395) (end 112.575 101.395) (width 0.3) (layer B.Cu) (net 21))
 (segment (start 112.575 101.395) (end 108.89 105.08) (width 0.3) (layer B.Cu) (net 21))
 (segment (start 125.5 103.935) (end 112.575 103.935) (width 0.3) (layer B.Cu) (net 22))
 (segment (start 112.575 103.935) (end 108.89 107.62) (width 0.3) (layer B.Cu) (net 22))
 (segment (start 125.625 111.485) (end 110.215 111.485) (width 0.3) (layer B.Cu) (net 23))
 (segment (start 110.215 111.485) (end 108.89 110.16) (width 0.3) (layer B.Cu) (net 23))
 (segment (start 108.89 112.7) (end 110.215 114.025) (width 0.3) (layer B.Cu) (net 24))
 (segment (start 110.215 114.025) (end 125.625 114.025) (width 0.3) (layer B.Cu) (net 24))
 (segment (start 125.5 98.855) (end 124.055 98.855) (width 0.3) (layer B.Cu) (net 4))
 (segment (start 119.475 90.675) (end 110.6 81.8) (width 0.3) (layer B.Cu) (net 4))
 (segment (start 124.055 98.855) (end 119.475 94.275) (width 0.3) (layer B.Cu) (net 4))
 (segment (start 119.475 94.275) (end 119.475 90.675) (width 0.3) (layer B.Cu) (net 4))
 (segment (start 110.6 81.8) (end 94.07 81.8) (width 0.3) (layer B.Cu) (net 4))
 (segment (start 94.07 81.8) (end 92.059999 83.810001) (width 0.3) (layer B.Cu) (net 4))
 (segment (start 92.059999 83.810001) (end 91.11 84.76) (width 0.3) (layer B.Cu) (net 4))
 (segment (start 78.925 105.2) (end 78.925 89.025) (width 0.3) (layer F.Cu) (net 4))
 (segment (start 80.399999 87.550001) (end 80.1 87.85) (width 0.3) (layer B.Cu) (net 4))
 (segment (start 83.19 84.76) (end 80.399999 87.550001) (width 0.3) (layer B.Cu) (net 4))
 (segment (start 79.800001 88.149999) (end 80.1 87.85) (width 0.3) (layer F.Cu) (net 4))
 (via (at 80.1 87.85) (size 0.6) (drill 0.4) (layers F.Cu B.Cu) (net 4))
 (segment (start 78.925 89.025) (end 79.800001 88.149999) (width 0.3) (layer F.Cu) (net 4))
 (segment (start 91.11 84.76) (end 83.19 84.76) (width 0.3) (layer B.Cu) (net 4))
 (segment (start 75.755 105.205) (end 75.9074 105.205) (width 0.3) (layer B.Cu) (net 4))
 (segment (start 75.9074 105.205) (end 75.9124 105.2) (width 0.3) (layer B.Cu) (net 4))
 (segment (start 75.9124 105.2) (end 78.925 105.2) (width 0.3) (layer B.Cu) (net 4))
 (via (at 78.925 105.2) (size 0.6) (drill 0.4) (layers F.Cu B.Cu) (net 4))
 (segment (start 125.625 116.565) (end 126.941 116.565) (width 0.3) (layer B.Cu) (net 4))
 (segment (start 126.941 116.565) (end 127.04101 116.46499) (width 0.3) (layer B.Cu) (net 4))
 (segment (start 127.04101 116.46499) (end 127.04101 100.24361) (width 0.3) (layer B.Cu) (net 4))
 (segment (start 127.04101 100.24361) (end 125.6524 98.855) (width 0.3) (layer B.Cu) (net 4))
 (segment (start 125.6524 98.855) (end 125.5 98.855) (width 0.3) (layer B.Cu) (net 4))
 (segment (start 75.755 105.205) (end 75.755 111.1624) (width 0.3) (layer B.Cu) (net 4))
 (segment (start 75.755 111.1624) (end 78.7726 114.18) (width 0.3) (layer B.Cu) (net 4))
 (segment (start 78.7726 114.18) (end 78.925 114.18) (width 0.3) (layer B.Cu) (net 4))
 (segment (start 90.4 84.05) (end 91.11 84.76) (width 0.3) (layer B.Cu) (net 4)))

